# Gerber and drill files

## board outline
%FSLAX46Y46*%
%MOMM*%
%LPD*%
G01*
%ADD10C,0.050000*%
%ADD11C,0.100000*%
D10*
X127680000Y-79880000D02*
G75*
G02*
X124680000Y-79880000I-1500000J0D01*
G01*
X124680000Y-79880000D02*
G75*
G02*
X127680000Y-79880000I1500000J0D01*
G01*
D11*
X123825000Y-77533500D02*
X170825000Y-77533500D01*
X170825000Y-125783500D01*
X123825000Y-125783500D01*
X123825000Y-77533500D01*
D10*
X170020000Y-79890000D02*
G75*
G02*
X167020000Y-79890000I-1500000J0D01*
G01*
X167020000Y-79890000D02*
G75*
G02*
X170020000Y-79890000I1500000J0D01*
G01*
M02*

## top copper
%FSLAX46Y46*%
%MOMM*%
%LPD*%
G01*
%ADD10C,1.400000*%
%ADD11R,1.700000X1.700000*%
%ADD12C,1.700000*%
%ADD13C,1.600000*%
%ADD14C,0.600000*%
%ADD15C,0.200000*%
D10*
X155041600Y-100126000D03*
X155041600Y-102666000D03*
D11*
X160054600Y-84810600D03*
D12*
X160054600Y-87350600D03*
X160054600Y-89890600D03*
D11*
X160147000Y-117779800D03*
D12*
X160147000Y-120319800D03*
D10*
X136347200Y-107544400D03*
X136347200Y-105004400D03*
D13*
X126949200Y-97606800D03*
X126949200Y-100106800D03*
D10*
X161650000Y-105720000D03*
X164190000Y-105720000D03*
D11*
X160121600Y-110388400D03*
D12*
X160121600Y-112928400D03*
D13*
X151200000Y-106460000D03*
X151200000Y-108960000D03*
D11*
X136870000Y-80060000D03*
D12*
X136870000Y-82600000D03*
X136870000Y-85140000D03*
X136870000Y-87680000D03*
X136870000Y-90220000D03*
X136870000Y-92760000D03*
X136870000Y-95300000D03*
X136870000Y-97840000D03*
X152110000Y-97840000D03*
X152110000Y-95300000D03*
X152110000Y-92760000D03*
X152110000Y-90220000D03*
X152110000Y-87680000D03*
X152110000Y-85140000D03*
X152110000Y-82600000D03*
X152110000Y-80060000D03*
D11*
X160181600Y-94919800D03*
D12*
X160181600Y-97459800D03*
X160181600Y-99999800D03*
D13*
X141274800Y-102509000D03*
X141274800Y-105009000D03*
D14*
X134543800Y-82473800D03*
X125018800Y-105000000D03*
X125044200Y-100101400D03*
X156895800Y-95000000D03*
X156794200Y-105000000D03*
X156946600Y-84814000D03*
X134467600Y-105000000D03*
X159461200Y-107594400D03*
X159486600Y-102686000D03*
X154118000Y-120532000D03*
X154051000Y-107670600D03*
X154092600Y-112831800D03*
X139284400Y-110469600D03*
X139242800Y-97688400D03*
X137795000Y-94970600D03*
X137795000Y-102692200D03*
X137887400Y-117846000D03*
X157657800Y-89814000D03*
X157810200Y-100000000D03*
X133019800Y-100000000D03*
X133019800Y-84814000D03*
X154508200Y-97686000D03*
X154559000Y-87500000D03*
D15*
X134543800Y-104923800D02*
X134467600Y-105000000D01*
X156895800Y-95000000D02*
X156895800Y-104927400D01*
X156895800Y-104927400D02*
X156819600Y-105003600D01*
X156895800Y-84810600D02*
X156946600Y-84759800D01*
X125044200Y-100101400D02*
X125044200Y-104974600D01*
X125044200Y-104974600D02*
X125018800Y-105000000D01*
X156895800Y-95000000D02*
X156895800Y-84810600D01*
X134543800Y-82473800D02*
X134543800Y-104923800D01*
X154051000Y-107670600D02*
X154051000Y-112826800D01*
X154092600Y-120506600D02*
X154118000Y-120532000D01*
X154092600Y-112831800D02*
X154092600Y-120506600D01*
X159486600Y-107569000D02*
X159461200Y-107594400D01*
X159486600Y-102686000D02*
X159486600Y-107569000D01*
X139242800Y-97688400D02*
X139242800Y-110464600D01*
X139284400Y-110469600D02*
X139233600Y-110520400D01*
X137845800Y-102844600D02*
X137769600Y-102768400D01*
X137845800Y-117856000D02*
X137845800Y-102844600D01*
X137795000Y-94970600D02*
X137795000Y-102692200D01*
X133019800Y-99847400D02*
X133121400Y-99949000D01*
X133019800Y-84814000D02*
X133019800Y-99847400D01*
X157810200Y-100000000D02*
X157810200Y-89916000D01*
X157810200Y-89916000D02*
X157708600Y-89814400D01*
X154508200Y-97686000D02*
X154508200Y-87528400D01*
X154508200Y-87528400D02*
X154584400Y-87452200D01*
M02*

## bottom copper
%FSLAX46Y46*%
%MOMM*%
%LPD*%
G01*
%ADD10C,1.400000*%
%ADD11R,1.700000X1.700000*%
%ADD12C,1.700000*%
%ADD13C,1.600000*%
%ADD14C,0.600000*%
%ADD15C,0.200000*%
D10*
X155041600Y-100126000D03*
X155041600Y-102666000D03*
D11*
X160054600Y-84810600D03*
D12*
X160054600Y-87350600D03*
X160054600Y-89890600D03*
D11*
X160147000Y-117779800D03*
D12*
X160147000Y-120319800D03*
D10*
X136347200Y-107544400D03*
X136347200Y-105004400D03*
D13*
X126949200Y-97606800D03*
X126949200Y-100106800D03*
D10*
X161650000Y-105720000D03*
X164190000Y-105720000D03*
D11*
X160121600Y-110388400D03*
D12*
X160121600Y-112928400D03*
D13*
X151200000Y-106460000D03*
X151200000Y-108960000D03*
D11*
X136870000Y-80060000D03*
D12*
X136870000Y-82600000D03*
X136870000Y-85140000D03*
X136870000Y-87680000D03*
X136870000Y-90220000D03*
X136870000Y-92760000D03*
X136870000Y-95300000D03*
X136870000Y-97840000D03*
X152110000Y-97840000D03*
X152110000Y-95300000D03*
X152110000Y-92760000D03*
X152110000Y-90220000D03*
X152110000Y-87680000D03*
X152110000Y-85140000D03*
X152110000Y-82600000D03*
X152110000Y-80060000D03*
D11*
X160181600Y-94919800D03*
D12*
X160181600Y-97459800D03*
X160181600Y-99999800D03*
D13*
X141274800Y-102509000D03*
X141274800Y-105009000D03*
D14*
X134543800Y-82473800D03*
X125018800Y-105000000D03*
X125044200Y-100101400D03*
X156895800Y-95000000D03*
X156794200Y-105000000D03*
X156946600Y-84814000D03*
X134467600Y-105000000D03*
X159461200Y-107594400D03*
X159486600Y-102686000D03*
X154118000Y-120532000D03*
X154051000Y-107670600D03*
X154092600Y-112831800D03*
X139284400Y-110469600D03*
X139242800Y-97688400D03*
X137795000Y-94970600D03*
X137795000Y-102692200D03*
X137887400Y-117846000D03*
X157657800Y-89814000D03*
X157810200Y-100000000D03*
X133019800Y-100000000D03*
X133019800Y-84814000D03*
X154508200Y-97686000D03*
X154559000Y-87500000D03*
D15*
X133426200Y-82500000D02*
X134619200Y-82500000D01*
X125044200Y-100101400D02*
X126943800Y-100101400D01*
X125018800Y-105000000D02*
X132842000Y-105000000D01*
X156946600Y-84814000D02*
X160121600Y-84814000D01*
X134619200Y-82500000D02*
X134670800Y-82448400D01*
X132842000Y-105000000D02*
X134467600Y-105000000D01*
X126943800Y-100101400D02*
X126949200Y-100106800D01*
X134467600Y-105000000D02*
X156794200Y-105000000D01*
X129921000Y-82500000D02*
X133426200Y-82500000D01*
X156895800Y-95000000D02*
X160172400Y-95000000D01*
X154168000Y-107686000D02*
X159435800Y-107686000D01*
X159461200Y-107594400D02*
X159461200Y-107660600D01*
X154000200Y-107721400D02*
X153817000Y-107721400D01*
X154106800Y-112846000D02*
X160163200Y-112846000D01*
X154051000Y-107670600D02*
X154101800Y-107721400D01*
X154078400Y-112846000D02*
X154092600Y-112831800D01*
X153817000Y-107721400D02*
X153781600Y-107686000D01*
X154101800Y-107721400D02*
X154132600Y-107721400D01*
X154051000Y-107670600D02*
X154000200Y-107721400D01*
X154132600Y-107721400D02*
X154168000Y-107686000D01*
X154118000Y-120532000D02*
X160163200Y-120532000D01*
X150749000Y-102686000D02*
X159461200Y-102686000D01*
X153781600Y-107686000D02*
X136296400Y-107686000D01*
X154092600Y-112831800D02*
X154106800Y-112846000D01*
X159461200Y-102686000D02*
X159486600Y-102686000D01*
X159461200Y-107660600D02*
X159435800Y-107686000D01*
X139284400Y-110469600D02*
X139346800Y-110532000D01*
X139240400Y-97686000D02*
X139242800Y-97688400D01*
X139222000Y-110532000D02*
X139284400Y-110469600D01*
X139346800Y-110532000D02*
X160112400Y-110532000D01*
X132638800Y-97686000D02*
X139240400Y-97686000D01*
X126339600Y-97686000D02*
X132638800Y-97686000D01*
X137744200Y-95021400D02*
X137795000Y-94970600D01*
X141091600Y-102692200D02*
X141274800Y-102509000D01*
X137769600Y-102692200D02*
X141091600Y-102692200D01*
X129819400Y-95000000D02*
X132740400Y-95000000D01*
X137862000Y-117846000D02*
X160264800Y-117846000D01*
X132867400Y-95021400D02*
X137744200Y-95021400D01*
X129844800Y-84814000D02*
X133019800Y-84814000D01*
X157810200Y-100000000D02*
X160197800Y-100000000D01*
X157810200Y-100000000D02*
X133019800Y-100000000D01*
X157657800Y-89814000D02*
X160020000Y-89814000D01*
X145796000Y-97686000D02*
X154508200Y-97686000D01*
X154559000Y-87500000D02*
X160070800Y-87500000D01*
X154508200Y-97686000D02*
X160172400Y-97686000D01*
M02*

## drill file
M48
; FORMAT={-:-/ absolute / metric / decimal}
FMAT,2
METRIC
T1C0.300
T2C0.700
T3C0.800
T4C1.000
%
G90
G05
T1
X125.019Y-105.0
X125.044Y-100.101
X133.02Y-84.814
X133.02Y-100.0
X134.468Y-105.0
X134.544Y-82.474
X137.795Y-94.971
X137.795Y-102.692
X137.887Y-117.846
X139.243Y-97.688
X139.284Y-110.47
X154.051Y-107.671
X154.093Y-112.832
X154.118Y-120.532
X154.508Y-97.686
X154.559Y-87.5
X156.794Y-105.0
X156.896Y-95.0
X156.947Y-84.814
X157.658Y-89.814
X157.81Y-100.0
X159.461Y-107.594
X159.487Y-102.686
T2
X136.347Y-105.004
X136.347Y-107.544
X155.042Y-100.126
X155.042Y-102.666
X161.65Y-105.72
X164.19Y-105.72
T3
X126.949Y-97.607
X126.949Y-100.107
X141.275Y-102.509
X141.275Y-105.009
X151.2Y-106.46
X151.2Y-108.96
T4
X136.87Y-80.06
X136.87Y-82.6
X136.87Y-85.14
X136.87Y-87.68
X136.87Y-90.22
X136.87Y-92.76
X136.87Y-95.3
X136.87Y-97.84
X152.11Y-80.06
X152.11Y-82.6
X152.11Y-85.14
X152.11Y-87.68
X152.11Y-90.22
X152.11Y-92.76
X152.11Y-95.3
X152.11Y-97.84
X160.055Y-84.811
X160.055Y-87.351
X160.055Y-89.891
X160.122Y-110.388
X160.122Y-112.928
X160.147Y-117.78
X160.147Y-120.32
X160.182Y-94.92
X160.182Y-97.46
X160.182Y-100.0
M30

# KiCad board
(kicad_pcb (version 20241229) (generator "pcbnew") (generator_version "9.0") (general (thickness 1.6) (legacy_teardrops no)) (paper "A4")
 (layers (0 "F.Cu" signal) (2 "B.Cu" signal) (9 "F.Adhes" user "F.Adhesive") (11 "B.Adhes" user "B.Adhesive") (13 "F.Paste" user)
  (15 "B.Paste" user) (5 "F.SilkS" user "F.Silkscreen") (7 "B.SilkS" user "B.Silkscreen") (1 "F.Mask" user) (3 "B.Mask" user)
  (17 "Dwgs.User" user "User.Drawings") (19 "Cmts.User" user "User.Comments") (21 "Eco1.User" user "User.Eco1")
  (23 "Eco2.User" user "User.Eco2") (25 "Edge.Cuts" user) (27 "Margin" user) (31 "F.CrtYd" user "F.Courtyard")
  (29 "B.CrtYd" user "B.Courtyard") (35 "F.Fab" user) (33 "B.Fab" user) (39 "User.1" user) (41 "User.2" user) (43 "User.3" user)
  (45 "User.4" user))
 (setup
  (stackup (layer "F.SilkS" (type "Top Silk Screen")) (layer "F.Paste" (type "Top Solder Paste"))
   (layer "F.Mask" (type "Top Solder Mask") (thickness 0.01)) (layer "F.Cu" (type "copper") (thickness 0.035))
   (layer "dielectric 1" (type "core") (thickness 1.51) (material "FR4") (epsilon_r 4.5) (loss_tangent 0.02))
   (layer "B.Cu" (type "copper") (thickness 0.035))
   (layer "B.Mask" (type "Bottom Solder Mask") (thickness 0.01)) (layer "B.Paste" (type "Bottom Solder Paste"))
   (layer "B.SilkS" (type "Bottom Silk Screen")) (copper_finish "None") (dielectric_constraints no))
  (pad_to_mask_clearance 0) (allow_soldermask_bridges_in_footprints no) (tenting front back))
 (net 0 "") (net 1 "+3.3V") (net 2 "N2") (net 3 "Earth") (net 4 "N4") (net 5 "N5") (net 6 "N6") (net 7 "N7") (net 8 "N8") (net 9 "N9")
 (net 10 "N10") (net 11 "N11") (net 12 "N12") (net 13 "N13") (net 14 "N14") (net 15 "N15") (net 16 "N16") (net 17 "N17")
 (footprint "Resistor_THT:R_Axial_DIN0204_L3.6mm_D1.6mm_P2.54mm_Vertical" (layer "F.Cu") (at 155.0416 100.126 -90)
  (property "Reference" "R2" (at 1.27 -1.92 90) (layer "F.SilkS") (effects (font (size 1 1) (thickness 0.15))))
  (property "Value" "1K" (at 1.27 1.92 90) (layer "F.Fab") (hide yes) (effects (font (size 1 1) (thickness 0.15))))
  (pad "1" thru_hole circle (at 0 0 270) (size 1.4 1.4) (drill 0.7) (layers "*.Cu" "*.Mask") (remove_unused_layers no) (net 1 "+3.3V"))
  (pad "2" thru_hole circle (at 2.54 0 270) (size 1.4 1.4) (drill 0.7) (layers "*.Cu" "*.Mask") (remove_unused_layers no) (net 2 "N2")))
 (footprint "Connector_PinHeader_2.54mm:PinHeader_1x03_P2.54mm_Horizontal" (layer "F.Cu") (at 160.0546 84.8106)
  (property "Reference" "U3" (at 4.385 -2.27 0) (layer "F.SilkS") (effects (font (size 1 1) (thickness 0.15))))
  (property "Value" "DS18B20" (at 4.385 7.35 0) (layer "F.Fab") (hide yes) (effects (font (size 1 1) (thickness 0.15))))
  (pad "1" thru_hole rect (at 0 0) (size 1.7 1.7) (drill 1) (layers "*.Cu" "*.Mask") (remove_unused_layers no) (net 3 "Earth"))
  (pad "2" thru_hole circle (at 0 2.54) (size 1.7 1.7) (drill 1) (layers "*.Cu" "*.Mask") (remove_unused_layers no) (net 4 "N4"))
  (pad "3" thru_hole circle (at 0 5.08) (size 1.7 1.7) (drill 1) (layers "*.Cu" "*.Mask") (remove_unused_layers no) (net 1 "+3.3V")))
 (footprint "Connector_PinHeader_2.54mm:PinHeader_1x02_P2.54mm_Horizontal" (layer "F.Cu") (at 160.147 117.7798)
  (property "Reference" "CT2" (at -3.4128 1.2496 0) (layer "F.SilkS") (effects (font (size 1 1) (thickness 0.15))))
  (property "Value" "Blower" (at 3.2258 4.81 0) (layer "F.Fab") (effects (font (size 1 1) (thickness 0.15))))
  (pad "1" thru_hole rect (at 0 0) (size 1.7 1.7) (drill 1) (layers "*.Cu" "*.Mask") (remove_unused_layers no) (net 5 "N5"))
  (pad "2" thru_hole circle (at 0 2.54) (size 1.7 1.7) (drill 1) (layers "*.Cu" "*.Mask") (remove_unused_layers no) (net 2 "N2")))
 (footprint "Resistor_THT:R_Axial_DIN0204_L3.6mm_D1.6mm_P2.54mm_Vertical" (layer "F.Cu") (at 136.3472 107.5444 90)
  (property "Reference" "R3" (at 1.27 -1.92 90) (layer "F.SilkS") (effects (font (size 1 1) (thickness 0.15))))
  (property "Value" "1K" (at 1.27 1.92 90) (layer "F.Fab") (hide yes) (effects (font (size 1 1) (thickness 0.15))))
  (pad "1" thru_hole circle (at 0 0 90) (size 1.4 1.4) (drill 0.7) (layers "*.Cu" "*.Mask") (remove_unused_layers no) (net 2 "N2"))
  (pad "2" thru_hole circle (at 2.54 0 90) (size 1.4 1.4) (drill 0.7) (layers "*.Cu" "*.Mask") (remove_unused_layers no) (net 3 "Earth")))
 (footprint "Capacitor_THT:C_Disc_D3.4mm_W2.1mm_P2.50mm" (layer "F.Cu") (at 126.9492 97.6068 -90)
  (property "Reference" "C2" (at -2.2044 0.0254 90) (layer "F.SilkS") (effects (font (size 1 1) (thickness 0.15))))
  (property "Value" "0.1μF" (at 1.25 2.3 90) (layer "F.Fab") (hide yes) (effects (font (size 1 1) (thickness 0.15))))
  (pad "1" thru_hole circle (at 0 0 270) (size 1.6 1.6) (drill 0.8) (layers "*.Cu" "*.Mask") (remove_unused_layers no) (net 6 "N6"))
  (pad "2" thru_hole circle (at 2.5 0 270) (size 1.6 1.6) (drill 0.8) (layers "*.Cu" "*.Mask") (remove_unused_layers no) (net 3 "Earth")))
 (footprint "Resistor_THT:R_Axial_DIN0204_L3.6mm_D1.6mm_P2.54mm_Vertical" (layer "F.Cu") (at 161.65 105.72)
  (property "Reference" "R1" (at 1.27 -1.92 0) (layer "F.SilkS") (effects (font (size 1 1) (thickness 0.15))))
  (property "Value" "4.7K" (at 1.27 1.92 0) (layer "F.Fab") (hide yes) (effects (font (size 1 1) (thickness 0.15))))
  (pad "1" thru_hole circle (at 0 0) (size 1.4 1.4) (drill 0.7) (layers "*.Cu" "*.Mask") (remove_unused_layers no) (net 1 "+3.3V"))
  (pad "2" thru_hole circle (at 2.54 0) (size 1.4 1.4) (drill 0.7) (layers "*.Cu" "*.Mask") (remove_unused_layers no) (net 4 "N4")))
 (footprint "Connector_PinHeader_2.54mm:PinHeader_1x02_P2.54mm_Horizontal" (layer "F.Cu") (at 160.1216 110.3884)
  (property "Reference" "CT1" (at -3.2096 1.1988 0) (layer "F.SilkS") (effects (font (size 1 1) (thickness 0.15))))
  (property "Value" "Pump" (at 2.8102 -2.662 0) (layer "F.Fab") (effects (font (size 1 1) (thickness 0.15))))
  (pad "1" thru_hole rect (at 0 0) (size 1.7 1.7) (drill 1) (layers "*.Cu" "*.Mask") (remove_unused_layers no) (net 6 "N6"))
  (pad "2" thru_hole circle (at 0 2.54) (size 1.7 1.7) (drill 1) (layers "*.Cu" "*.Mask") (remove_unused_layers no) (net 2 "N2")))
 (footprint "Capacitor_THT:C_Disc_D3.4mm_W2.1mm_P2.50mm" (layer "F.Cu") (at 151.2 106.46 -90)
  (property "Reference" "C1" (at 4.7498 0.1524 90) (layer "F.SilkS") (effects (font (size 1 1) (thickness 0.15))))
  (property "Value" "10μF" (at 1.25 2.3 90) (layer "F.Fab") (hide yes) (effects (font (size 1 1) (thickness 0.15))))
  (pad "1" thru_hole circle (at 0 0 270) (size 1.6 1.6) (drill 0.8) (layers "*.Cu" "*.Mask") (remove_unused_layers no) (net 2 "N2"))
  (pad "2" thru_hole circle (at 2.5 0 270) (size 1.6 1.6) (drill 0.8) (layers "*.Cu" "*.Mask") (remove_unused_layers no) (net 3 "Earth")))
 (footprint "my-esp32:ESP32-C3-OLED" (layer "F.Cu") (at 144.49 88.95)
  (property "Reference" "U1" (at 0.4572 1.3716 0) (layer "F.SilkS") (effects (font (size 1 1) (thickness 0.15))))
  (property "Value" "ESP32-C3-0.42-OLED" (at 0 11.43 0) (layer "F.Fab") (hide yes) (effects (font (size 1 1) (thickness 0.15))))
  (pad "1" thru_hole rect (at -7.62 -8.89) (size 1.7 1.7) (drill 1) (layers "*.Cu" "*.Mask") (remove_unused_layers no) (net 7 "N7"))
  (pad "2" thru_hole circle (at -7.62 -6.35) (size 1.7 1.7) (drill 1) (layers "*.Cu" "*.Mask") (remove_unused_layers no) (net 3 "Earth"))
  (pad "3" thru_hole circle (at -7.62 -3.81) (size 1.7 1.7) (drill 1) (layers "*.Cu" "*.Mask") (remove_unused_layers no) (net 1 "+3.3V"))
  (pad "4" thru_hole circle (at -7.62 -1.27) (size 1.7 1.7) (drill 1) (layers "*.Cu" "*.Mask") (remove_unused_layers no) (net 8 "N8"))
  (pad "5" thru_hole circle (at -7.62 1.27) (size 1.7 1.7) (drill 1) (layers "*.Cu" "*.Mask") (remove_unused_layers no) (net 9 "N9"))
  (pad "6" thru_hole circle (at -7.62 3.81) (size 1.7 1.7) (drill 1) (layers "*.Cu" "*.Mask") (remove_unused_layers no) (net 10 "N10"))
  (pad "7" thru_hole circle (at -7.62 6.35) (size 1.7 1.7) (drill 1) (layers "*.Cu" "*.Mask") (remove_unused_layers no) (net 5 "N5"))
  (pad "8" thru_hole circle (at -7.62 8.89) (size 1.7 1.7) (drill 1) (layers "*.Cu" "*.Mask") (remove_unused_layers no) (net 6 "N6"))
  (pad "9" thru_hole circle (at 7.62 8.89) (size 1.7 1.7) (drill 1) (layers "*.Cu" "*.Mask") (remove_unused_layers no) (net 4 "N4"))
  (pad "10" thru_hole circle (at 7.62 6.35) (size 1.7 1.7) (drill 1) (layers "*.Cu" "*.Mask") (remove_unused_layers no) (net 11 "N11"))
  (pad "11" thru_hole circle (at 7.62 3.81) (size 1.7 1.7) (drill 1) (layers "*.Cu" "*.Mask") (remove_unused_layers no) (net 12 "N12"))
  (pad "12" thru_hole circle (at 7.62 1.27) (size 1.7 1.7) (drill 1) (layers "*.Cu" "*.Mask") (remove_unused_layers no) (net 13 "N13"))
  (pad "13" thru_hole circle (at 7.62 -1.27) (size 1.7 1.7) (drill 1) (layers "*.Cu" "*.Mask") (remove_unused_layers no) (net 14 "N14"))
  (pad "14" thru_hole circle (at 7.62 -3.81) (size 1.7 1.7) (drill 1) (layers "*.Cu" "*.Mask") (remove_unused_layers no) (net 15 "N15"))
  (pad "15" thru_hole circle (at 7.62 -6.35) (size 1.7 1.7) (drill 1) (layers "*.Cu" "*.Mask") (remove_unused_layers no) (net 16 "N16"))
  (pad "16" thru_hole circle (at 7.62 -8.89) (size 1.7 1.7) (drill 1) (layers "*.Cu" "*.Mask") (remove_unused_layers no) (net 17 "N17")))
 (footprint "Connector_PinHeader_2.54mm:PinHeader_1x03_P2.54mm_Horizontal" (layer "F.Cu") (at 160.1816 94.9198)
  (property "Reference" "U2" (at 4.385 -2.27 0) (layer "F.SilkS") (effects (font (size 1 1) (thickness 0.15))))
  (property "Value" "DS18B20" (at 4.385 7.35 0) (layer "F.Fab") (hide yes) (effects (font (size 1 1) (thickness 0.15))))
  (pad "1" thru_hole rect (at 0 0) (size 1.7 1.7) (drill 1) (layers "*.Cu" "*.Mask") (remove_unused_layers no) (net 3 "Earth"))
  (pad "2" thru_hole circle (at 0 2.54) (size 1.7 1.7) (drill 1) (layers "*.Cu" "*.Mask") (remove_unused_layers no) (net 4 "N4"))
  (pad "3" thru_hole circle (at 0 5.08) (size 1.7 1.7) (drill 1) (layers "*.Cu" "*.Mask") (remove_unused_layers no) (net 1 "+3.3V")))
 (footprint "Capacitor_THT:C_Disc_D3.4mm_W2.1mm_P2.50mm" (layer "F.Cu") (at 141.2748 102.509 -90)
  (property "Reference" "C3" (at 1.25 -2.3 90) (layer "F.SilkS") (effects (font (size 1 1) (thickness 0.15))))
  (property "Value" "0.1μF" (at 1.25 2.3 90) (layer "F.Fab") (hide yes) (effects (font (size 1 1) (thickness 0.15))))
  (pad "1" thru_hole circle (at 0 0 270) (size 1.6 1.6) (drill 0.8) (layers "*.Cu" "*.Mask") (remove_unused_layers no) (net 5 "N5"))
  (pad "2" thru_hole circle (at 2.5 0 270) (size 1.6 1.6) (drill 0.8) (layers "*.Cu" "*.Mask") (remove_unused_layers no) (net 3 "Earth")))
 (gr_circle (center 126.18 79.88) (end 127.68 79.88) (stroke (width 0.05) (type solid)) (fill no) (layer "Edge.Cuts"))
 (gr_rect (start 123.825 77.5335) (end 170.825 125.7835) (stroke (width 0.1) (type solid)) (fill no) (layer "Edge.Cuts"))
 (gr_circle (center 168.52 79.89) (end 170.02 79.89) (stroke (width 0.05) (type solid)) (fill no) (layer "Edge.Cuts"))
 (segment (start 134.5438 104.9238) (end 134.4676 105) (width 0.2) (layer "F.Cu") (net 3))
 (segment (start 156.8958 95) (end 156.8958 104.9274) (width 0.2) (layer "F.Cu") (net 3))
 (segment (start 156.8958 104.9274) (end 156.8196 105.0036) (width 0.2) (layer "F.Cu") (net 3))
 (segment (start 156.8958 84.8106) (end 156.9466 84.7598) (width 0.2) (layer "F.Cu") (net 3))
 (segment (start 125.0442 100.1014) (end 125.0442 104.9746) (width 0.2) (layer "F.Cu") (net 3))
 (segment (start 125.0442 104.9746) (end 125.0188 105) (width 0.2) (layer "F.Cu") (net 3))
 (segment (start 156.8958 95) (end 156.8958 84.8106) (width 0.2) (layer "F.Cu") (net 3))
 (segment (start 134.5438 82.4738) (end 134.5438 104.9238) (width 0.2) (layer "F.Cu") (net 3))
 (via (at 134.5438 82.4738) (size 0.6) (drill 0.3) (layers "F.Cu" "B.Cu") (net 3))
 (via (at 125.0188 105) (size 0.6) (drill 0.3) (layers "F.Cu" "B.Cu") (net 3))
 (via (at 125.0442 100.1014) (size 0.6) (drill 0.3) (layers "F.Cu" "B.Cu") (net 3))
 (via (at 156.8958 95) (size 0.6) (drill 0.3) (layers "F.Cu" "B.Cu") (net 3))
 (via (at 156.7942 105) (size 0.6) (drill 0.3) (layers "F.Cu" "B.Cu") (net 3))
 (via (at 156.9466 84.814) (size 0.6) (drill 0.3) (layers "F.Cu" "B.Cu") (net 3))
 (via (at 134.4676 105) (size 0.6) (drill 0.3) (layers "F.Cu" "B.Cu") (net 3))
 (segment (start 133.4262 82.5) (end 134.6192 82.5) (width 0.2) (layer "B.Cu") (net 3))
 (segment (start 125.0442 100.1014) (end 126.9438 100.1014) (width 0.2) (layer "B.Cu") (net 3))
 (segment (start 125.0188 105) (end 132.842 105) (width 0.2) (layer "B.Cu") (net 3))
 (segment (start 156.9466 84.814) (end 160.1216 84.814) (width 0.2) (layer "B.Cu") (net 3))
 (segment (start 134.6192 82.5) (end 134.6708 82.4484) (width 0.2) (layer "B.Cu") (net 3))
 (segment (start 132.842 105) (end 134.4676 105) (width 0.2) (layer "B.Cu") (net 3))
 (segment (start 126.9438 100.1014) (end 126.9492 100.1068) (width 0.2) (layer "B.Cu") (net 3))
 (segment (start 134.4676 105) (end 156.7942 105) (width 0.2) (layer "B.Cu") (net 3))
 (segment (start 129.921 82.5) (end 133.4262 82.5) (width 0.2) (layer "B.Cu") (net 3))
 (segment (start 156.8958 95) (end 160.1724 95) (width 0.2) (layer "B.Cu") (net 3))
 (segment (start 154.051 107.6706) (end 154.051 112.8268) (width 0.2) (layer "F.Cu") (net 2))
 (segment (start 154.0926 120.5066) (end 154.118 120.532) (width 0.2) (layer "F.Cu") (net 2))
 (segment (start 154.0926 112.8318) (end 154.0926 120.5066) (width 0.2) (layer "F.Cu") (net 2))
 (segment (start 159.4866 107.569) (end 159.4612 107.5944) (width 0.2) (layer "F.Cu") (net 2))
 (segment (start 159.4866 102.686) (end 159.4866 107.569) (width 0.2) (layer "F.Cu") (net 2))
 (via (at 159.4612 107.5944) (size 0.6) (drill 0.3) (layers "F.Cu" "B.Cu") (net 2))
 (via (at 159.4866 102.686) (size 0.6) (drill 0.3) (layers "F.Cu" "B.Cu") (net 2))
 (via (at 154.118 120.532) (size 0.6) (drill 0.3) (layers "F.Cu" "B.Cu") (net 2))
 (via (at 154.051 107.6706) (size 0.6) (drill 0.3) (layers "F.Cu" "B.Cu") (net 2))
 (via (at 154.0926 112.8318) (size 0.6) (drill 0.3) (layers "F.Cu" "B.Cu") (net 2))
 (segment (start 154.168 107.686) (end 159.4358 107.686) (width 0.2) (layer "B.Cu") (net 2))
 (segment (start 159.4612 107.5944) (end 159.4612 107.6606) (width 0.2) (layer "B.Cu") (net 2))
 (segment (start 154.0002 107.7214) (end 153.817 107.7214) (width 0.2) (layer "B.Cu") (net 2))
 (segment (start 154.1068 112.846) (end 160.1632 112.846) (width 0.2) (layer "B.Cu") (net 2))
 (segment (start 154.051 107.6706) (end 154.1018 107.7214) (width 0.2) (layer "B.Cu") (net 2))
 (segment (start 154.0784 112.846) (end 154.0926 112.8318) (width 0.2) (layer "B.Cu") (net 2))
 (segment (start 153.817 107.7214) (end 153.7816 107.686) (width 0.2) (layer "B.Cu") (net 2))
 (segment (start 154.1018 107.7214) (end 154.1326 107.7214) (width 0.2) (layer "B.Cu") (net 2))
 (segment (start 154.051 107.6706) (end 154.0002 107.7214) (width 0.2) (layer "B.Cu") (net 2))
 (segment (start 154.1326 107.7214) (end 154.168 107.686) (width 0.2) (layer "B.Cu") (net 2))
 (segment (start 154.118 120.532) (end 160.1632 120.532) (width 0.2) (layer "B.Cu") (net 2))
 (segment (start 150.749 102.686) (end 159.4612 102.686) (width 0.2) (layer "B.Cu") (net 2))
 (segment (start 153.7816 107.686) (end 136.2964 107.686) (width 0.2) (layer "B.Cu") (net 2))
 (segment (start 154.0926 112.8318) (end 154.1068 112.846) (width 0.2) (layer "B.Cu") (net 2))
 (segment (start 159.4612 102.686) (end 159.4866 102.686) (width 0.2) (layer "B.Cu") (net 2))
 (segment (start 159.4612 107.6606) (end 159.4358 107.686) (width 0.2) (layer "B.Cu") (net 2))
 (segment (start 139.2428 97.6884) (end 139.2428 110.4646) (width 0.2) (layer "F.Cu") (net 6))
 (segment (start 139.2844 110.4696) (end 139.2336 110.5204) (width 0.2) (layer "F.Cu") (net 6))
 (via (at 139.2844 110.4696) (size 0.6) (drill 0.3) (layers "F.Cu" "B.Cu") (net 6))
 (via (at 139.2428 97.6884) (size 0.6) (drill 0.3) (layers "F.Cu" "B.Cu") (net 6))
 (segment (start 139.2844 110.4696) (end 139.3468 110.532) (width 0.2) (layer "B.Cu") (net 6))
 (segment (start 139.2404 97.686) (end 139.2428 97.6884) (width 0.2) (layer "B.Cu") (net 6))
 (segment (start 139.222 110.532) (end 139.2844 110.4696) (width 0.2) (layer "B.Cu") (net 6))
 (segment (start 139.3468 110.532) (end 160.1124 110.532) (width 0.2) (layer "B.Cu") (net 6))
 (segment (start 132.6388 97.686) (end 139.2404 97.686) (width 0.2) (layer "B.Cu") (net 6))
 (segment (start 126.3396 97.686) (end 132.6388 97.686) (width 0.2) (layer "B.Cu") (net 6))
 (segment (start 137.8458 102.8446) (end 137.7696 102.7684) (width 0.2) (layer "F.Cu") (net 5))
 (segment (start 137.8458 117.856) (end 137.8458 102.8446) (width 0.2) (layer "F.Cu") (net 5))
 (segment (start 137.795 94.9706) (end 137.795 102.6922) (width 0.2) (layer "F.Cu") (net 5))
 (via (at 137.795 94.9706) (size 0.6) (drill 0.3) (layers "F.Cu" "B.Cu") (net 5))
 (via (at 137.795 102.6922) (size 0.6) (drill 0.3) (layers "F.Cu" "B.Cu") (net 5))
 (via (at 137.8874 117.846) (size 0.6) (drill 0.3) (layers "F.Cu" "B.Cu") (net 5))
 (segment (start 137.7442 95.0214) (end 137.795 94.9706) (width 0.2) (layer "B.Cu") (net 5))
 (segment (start 141.0916 102.6922) (end 141.2748 102.509) (width 0.2) (layer "B.Cu") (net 5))
 (segment (start 137.7696 102.6922) (end 141.0916 102.6922) (width 0.2) (layer "B.Cu") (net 5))
 (segment (start 129.8194 95) (end 132.7404 95) (width 0.2) (layer "B.Cu") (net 5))
 (segment (start 137.862 117.846) (end 160.2648 117.846) (width 0.2) (layer "B.Cu") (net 5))
 (segment (start 132.8674 95.0214) (end 137.7442 95.0214) (width 0.2) (layer "B.Cu") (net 5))
 (segment (start 133.0198 99.8474) (end 133.1214 99.949) (width 0.2) (layer "F.Cu") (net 1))
 (segment (start 133.0198 84.814) (end 133.0198 99.8474) (width 0.2) (layer "F.Cu") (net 1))
 (segment (start 157.8102 100) (end 157.8102 89.916) (width 0.2) (layer "F.Cu") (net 1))
 (segment (start 157.8102 89.916) (end 157.7086 89.8144) (width 0.2) (layer "F.Cu") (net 1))
 (via (at 157.6578 89.814) (size 0.6) (drill 0.3) (layers "F.Cu" "B.Cu") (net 1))
 (via (at 157.8102 100) (size 0.6) (drill 0.3) (layers "F.Cu" "B.Cu") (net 1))
 (via (at 133.0198 100) (size 0.6) (drill 0.3) (layers "F.Cu" "B.Cu") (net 1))
 (via (at 133.0198 84.814) (size 0.6) (drill 0.3) (layers "F.Cu" "B.Cu") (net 1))
 (segment (start 129.8448 84.814) (end 133.0198 84.814) (width 0.2) (layer "B.Cu") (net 1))
 (segment (start 157.8102 100) (end 160.1978 100) (width 0.2) (layer "B.Cu") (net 1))
 (segment (start 157.8102 100) (end 133.0198 100) (width 0.2) (layer "B.Cu") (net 1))
 (segment (start 157.6578 89.814) (end 160.02 89.814) (width 0.2) (layer "B.Cu") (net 1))
 (segment (start 154.5082 97.686) (end 154.5082 87.5284) (width 0.2) (layer "F.Cu") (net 4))
 (segment (start 154.5082 87.5284) (end 154.5844 87.4522) (width 0.2) (layer "F.Cu") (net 4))
 (via (at 154.5082 97.686) (size 0.6) (drill 0.3) (layers "F.Cu" "B.Cu") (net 4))
 (via (at 154.559 87.5) (size 0.6) (drill 0.3) (layers "F.Cu" "B.Cu") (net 4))
 (segment (start 145.796 97.686) (end 154.5082 97.686) (width 0.2) (layer "B.Cu") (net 4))
 (segment (start 154.559 87.5) (end 160.0708 87.5) (width 0.2) (layer "B.Cu") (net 4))
 (segment (start 154.5082 97.686) (end 160.1724 97.686) (width 0.2) (layer "B.Cu") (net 4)))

